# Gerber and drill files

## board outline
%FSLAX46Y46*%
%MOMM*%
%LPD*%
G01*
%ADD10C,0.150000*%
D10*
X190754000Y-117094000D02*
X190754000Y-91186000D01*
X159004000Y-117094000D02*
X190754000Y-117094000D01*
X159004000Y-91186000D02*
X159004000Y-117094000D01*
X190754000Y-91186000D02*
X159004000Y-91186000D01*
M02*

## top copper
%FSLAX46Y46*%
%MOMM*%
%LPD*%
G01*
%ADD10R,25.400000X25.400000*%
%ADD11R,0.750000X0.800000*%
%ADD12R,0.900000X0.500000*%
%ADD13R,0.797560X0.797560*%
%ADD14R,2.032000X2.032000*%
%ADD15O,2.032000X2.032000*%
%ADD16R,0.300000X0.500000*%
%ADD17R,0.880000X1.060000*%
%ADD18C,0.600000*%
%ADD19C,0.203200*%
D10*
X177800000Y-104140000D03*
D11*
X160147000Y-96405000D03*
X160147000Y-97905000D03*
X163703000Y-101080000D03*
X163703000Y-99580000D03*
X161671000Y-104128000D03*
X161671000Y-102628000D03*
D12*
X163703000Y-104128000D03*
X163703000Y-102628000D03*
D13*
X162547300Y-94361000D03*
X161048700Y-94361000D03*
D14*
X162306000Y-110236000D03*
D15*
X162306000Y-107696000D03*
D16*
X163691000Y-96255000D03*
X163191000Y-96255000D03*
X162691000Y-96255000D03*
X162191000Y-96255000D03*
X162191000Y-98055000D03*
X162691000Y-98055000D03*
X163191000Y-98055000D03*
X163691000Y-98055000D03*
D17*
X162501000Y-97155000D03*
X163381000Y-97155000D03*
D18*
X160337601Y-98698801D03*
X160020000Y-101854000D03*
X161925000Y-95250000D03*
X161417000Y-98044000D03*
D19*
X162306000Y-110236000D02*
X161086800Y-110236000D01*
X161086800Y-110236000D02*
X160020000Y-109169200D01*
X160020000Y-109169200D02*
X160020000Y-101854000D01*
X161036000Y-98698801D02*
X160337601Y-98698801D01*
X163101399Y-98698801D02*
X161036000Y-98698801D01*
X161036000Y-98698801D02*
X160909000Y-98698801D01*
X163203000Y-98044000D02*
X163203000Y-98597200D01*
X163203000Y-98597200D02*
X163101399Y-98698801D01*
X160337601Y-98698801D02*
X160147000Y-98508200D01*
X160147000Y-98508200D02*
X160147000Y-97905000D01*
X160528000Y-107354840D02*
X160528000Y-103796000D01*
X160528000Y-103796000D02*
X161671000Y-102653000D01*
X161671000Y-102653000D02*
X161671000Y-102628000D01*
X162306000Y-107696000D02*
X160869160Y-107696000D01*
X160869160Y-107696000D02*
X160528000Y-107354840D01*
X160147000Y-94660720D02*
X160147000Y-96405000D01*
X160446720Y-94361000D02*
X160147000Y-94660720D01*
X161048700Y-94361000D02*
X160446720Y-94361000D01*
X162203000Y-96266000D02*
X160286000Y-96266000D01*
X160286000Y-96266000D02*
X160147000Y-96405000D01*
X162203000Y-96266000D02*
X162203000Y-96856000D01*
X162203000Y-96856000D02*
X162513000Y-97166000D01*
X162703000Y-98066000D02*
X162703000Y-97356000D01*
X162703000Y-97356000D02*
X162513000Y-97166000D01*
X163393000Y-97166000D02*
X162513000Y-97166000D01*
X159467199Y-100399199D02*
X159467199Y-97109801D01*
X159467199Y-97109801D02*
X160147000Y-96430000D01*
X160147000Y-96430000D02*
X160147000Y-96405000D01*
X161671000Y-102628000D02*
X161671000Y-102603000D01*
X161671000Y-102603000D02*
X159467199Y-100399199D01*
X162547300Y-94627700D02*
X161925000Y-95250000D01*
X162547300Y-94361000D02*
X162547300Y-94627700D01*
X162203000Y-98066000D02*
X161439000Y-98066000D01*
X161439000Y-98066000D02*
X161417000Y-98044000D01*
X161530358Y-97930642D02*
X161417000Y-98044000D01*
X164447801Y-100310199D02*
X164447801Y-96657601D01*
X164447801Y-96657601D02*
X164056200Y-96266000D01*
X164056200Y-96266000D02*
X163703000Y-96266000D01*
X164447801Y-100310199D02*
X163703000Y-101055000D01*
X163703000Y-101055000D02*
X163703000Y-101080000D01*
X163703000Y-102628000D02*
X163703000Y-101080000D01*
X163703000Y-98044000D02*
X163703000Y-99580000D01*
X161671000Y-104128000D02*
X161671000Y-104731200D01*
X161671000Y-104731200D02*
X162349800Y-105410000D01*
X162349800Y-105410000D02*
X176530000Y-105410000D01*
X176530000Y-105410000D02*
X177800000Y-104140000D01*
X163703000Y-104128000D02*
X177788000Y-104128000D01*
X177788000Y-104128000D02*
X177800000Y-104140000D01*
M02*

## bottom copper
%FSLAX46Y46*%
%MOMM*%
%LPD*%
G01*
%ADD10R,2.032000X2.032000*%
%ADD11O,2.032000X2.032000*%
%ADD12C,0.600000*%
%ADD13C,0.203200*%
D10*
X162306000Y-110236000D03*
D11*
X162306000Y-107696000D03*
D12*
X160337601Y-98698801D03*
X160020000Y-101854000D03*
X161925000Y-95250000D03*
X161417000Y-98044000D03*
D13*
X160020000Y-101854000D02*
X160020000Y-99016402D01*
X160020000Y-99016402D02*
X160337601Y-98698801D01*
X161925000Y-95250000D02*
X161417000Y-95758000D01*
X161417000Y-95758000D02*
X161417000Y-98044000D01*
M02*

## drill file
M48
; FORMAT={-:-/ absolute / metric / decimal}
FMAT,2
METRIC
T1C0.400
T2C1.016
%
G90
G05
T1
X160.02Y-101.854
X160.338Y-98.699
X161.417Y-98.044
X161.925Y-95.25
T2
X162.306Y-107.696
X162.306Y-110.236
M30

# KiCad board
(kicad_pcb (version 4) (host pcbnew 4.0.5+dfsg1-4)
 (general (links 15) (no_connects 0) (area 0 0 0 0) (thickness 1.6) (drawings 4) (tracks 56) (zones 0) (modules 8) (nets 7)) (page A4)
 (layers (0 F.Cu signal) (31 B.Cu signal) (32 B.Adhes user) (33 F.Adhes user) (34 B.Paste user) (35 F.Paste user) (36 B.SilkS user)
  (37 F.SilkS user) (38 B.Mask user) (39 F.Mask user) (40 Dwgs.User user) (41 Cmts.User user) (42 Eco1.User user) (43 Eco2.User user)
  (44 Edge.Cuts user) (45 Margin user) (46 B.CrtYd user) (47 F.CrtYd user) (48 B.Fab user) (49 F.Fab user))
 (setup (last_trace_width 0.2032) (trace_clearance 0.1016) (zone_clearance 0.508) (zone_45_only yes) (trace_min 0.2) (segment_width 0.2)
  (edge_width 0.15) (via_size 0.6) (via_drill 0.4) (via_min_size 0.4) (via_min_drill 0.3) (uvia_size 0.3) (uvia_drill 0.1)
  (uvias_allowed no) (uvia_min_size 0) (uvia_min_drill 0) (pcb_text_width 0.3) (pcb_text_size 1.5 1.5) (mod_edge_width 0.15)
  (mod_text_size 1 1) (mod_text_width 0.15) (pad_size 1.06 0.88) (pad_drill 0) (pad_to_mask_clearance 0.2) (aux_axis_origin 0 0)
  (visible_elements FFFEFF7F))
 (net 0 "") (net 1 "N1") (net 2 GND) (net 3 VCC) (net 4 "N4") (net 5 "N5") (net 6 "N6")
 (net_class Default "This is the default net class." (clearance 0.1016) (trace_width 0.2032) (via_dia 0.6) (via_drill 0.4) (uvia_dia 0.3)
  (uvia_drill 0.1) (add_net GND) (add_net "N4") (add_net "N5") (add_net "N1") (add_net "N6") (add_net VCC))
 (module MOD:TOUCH (layer F.Cu) (at 177.8 104.14)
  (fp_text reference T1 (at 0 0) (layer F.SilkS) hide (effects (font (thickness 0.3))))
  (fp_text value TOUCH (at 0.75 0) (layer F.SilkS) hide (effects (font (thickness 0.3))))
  (pad 1 connect rect (at 0 0) (size 25.4 25.4) (layers F.Cu) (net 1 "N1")))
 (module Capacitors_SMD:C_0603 (layer F.Cu) (at 160.147 97.155 270)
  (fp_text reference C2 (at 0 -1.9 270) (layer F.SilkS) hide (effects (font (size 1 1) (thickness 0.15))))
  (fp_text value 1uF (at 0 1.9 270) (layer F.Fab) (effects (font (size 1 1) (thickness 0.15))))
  (pad 1 smd rect (at -0.75 0 270) (size 0.8 0.75) (layers F.Cu F.Paste F.Mask) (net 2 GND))
  (pad 2 smd rect (at 0.75 0 270) (size 0.8 0.75) (layers F.Cu F.Paste F.Mask) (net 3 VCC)))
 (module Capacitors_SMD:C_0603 (layer F.Cu) (at 163.703 100.33 90)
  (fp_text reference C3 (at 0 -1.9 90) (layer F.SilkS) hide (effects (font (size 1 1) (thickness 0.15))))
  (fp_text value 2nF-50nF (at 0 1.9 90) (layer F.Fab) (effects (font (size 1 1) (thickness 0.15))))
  (pad 1 smd rect (at -0.75 0 90) (size 0.8 0.75) (layers F.Cu F.Paste F.Mask) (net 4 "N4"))
  (pad 2 smd rect (at 0.75 0 90) (size 0.8 0.75) (layers F.Cu F.Paste F.Mask) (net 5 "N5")))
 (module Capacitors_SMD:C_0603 (layer F.Cu) (at 161.671 103.378 90)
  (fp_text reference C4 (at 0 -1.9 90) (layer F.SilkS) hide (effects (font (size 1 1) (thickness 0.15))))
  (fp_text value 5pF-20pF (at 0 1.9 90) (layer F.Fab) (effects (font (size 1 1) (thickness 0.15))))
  (pad 1 smd rect (at -0.75 0 90) (size 0.8 0.75) (layers F.Cu F.Paste F.Mask) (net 1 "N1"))
  (pad 2 smd rect (at 0.75 0 90) (size 0.8 0.75) (layers F.Cu F.Paste F.Mask) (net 2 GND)))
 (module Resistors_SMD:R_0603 (layer F.Cu) (at 163.703 103.378 90)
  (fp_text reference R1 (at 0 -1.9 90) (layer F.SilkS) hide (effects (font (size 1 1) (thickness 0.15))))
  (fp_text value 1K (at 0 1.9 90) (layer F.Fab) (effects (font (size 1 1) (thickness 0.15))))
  (pad 1 smd rect (at -0.75 0 90) (size 0.5 0.9) (layers F.Cu F.Paste F.Mask) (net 1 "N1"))
  (pad 2 smd rect (at 0.75 0 90) (size 0.5 0.9) (layers F.Cu F.Paste F.Mask) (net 4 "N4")))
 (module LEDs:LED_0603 (layer F.Cu) (at 161.798 94.361)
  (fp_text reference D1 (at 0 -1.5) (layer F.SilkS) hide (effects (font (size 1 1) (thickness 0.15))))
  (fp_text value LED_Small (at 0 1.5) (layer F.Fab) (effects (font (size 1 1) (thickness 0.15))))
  (pad 2 smd rect (at 0.7493 0 180) (size 0.79756 0.79756) (layers F.Cu F.Paste F.Mask) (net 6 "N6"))
  (pad 1 smd rect (at -0.7493 0 180) (size 0.79756 0.79756) (layers F.Cu F.Paste F.Mask) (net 2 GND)))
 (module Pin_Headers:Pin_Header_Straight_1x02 (layer F.Cu) (at 162.306 110.236 180)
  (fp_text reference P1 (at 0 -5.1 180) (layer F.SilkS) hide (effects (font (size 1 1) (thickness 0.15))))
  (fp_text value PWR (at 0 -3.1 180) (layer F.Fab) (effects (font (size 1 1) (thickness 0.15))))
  (pad 1 thru_hole rect (at 0 0 180) (size 2.032 2.032) (drill 1.016) (layers *.Cu *.Mask) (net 3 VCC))
  (pad 2 thru_hole oval (at 0 2.54 180) (size 2.032 2.032) (drill 1.016) (layers *.Cu *.Mask) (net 2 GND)))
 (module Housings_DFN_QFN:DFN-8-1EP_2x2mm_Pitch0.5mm (layer F.Cu) (at 162.941 97.155 270)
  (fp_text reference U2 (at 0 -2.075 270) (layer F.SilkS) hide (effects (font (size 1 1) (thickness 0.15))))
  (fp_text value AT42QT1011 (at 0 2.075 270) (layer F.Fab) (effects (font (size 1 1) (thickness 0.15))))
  (pad 1 smd rect (at -0.9 -0.75 270) (size 0.5 0.3) (layers F.Cu F.Paste F.Mask) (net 4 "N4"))
  (pad 2 smd rect (at -0.9 -0.25 270) (size 0.5 0.3) (layers F.Cu F.Paste F.Mask))
  (pad 3 smd rect (at -0.9 0.25 270) (size 0.5 0.3) (layers F.Cu F.Paste F.Mask))
  (pad 4 smd rect (at -0.9 0.75 270) (size 0.5 0.3) (layers F.Cu F.Paste F.Mask) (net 2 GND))
  (pad 5 smd rect (at 0.9 0.75 270) (size 0.5 0.3) (layers F.Cu F.Paste F.Mask) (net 6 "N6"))
  (pad 6 smd rect (at 0.9 0.25 270) (size 0.5 0.3) (layers F.Cu F.Paste F.Mask) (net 2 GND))
  (pad 7 smd rect (at 0.9 -0.25 270) (size 0.5 0.3) (layers F.Cu F.Paste F.Mask) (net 3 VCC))
  (pad 8 smd rect (at 0.9 -0.75 270) (size 0.5 0.3) (layers F.Cu F.Paste F.Mask) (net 5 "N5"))
  (pad 9 smd rect (at 0 0.44 270) (size 1.06 0.88) (layers F.Cu F.Paste F.Mask) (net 2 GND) (solder_paste_margin_ratio -0.2))
  (pad 9 smd rect (at 0 -0.44 270) (size 1.06 0.88) (layers F.Cu F.Paste F.Mask) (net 2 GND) (solder_paste_margin_ratio -0.2)))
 (gr_line (start 190.754 117.094) (end 190.754 91.186) (layer Edge.Cuts) (width 0.15))
 (gr_line (start 159.004 117.094) (end 190.754 117.094) (layer Edge.Cuts) (width 0.15))
 (gr_line (start 159.004 91.186) (end 159.004 117.094) (layer Edge.Cuts) (width 0.15))
 (gr_line (start 190.754 91.186) (end 159.004 91.186) (layer Edge.Cuts) (width 0.15))
 (segment (start 160.02 101.854) (end 160.02 99.016402) (width 0.2032) (layer B.Cu) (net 3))
 (segment (start 160.02 99.016402) (end 160.337601 98.698801) (width 0.2032) (layer B.Cu) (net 3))
 (via (at 160.337601 98.698801) (size 0.6) (drill 0.4) (layers F.Cu B.Cu) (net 3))
 (segment (start 162.306 110.236) (end 161.0868 110.236) (width 0.2032) (layer F.Cu) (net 3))
 (segment (start 161.0868 110.236) (end 160.02 109.1692) (width 0.2032) (layer F.Cu) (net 3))
 (segment (start 160.02 109.1692) (end 160.02 101.854) (width 0.2032) (layer F.Cu) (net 3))
 (via (at 160.02 101.854) (size 0.6) (drill 0.4) (layers F.Cu B.Cu) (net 3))
 (segment (start 161.036 98.698801) (end 160.337601 98.698801) (width 0.2032) (layer F.Cu) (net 3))
 (segment (start 163.101399 98.698801) (end 161.036 98.698801) (width 0.2032) (layer F.Cu) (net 3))
 (segment (start 161.036 98.698801) (end 160.909 98.698801) (width 0.2032) (layer F.Cu) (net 3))
 (segment (start 163.203 98.044) (end 163.203 98.5972) (width 0.2032) (layer F.Cu) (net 3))
 (segment (start 163.203 98.5972) (end 163.101399 98.698801) (width 0.2032) (layer F.Cu) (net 3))
 (segment (start 160.337601 98.698801) (end 160.147 98.5082) (width 0.2032) (layer F.Cu) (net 3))
 (segment (start 160.147 98.5082) (end 160.147 97.905) (width 0.2032) (layer F.Cu) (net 3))
 (segment (start 160.528 107.35484) (end 160.528 103.796) (width 0.2032) (layer F.Cu) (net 2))
 (segment (start 160.528 103.796) (end 161.671 102.653) (width 0.2032) (layer F.Cu) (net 2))
 (segment (start 161.671 102.653) (end 161.671 102.628) (width 0.2032) (layer F.Cu) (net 2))
 (segment (start 162.306 107.696) (end 160.86916 107.696) (width 0.2032) (layer F.Cu) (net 2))
 (segment (start 160.86916 107.696) (end 160.528 107.35484) (width 0.2032) (layer F.Cu) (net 2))
 (segment (start 160.147 94.66072) (end 160.147 96.405) (width 0.2032) (layer F.Cu) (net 2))
 (segment (start 160.44672 94.361) (end 160.147 94.66072) (width 0.2032) (layer F.Cu) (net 2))
 (segment (start 161.0487 94.361) (end 160.44672 94.361) (width 0.2032) (layer F.Cu) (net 2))
 (segment (start 162.203 96.266) (end 160.286 96.266) (width 0.2032) (layer F.Cu) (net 2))
 (segment (start 160.286 96.266) (end 160.147 96.405) (width 0.2032) (layer F.Cu) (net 2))
 (segment (start 162.203 96.266) (end 162.203 96.856) (width 0.2032) (layer F.Cu) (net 2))
 (segment (start 162.203 96.856) (end 162.513 97.166) (width 0.2032) (layer F.Cu) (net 2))
 (segment (start 162.703 98.066) (end 162.703 97.356) (width 0.2032) (layer F.Cu) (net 2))
 (segment (start 162.703 97.356) (end 162.513 97.166) (width 0.2032) (layer F.Cu) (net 2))
 (segment (start 163.393 97.166) (end 162.513 97.166) (width 0.2032) (layer F.Cu) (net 2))
 (segment (start 159.467199 100.399199) (end 159.467199 97.109801) (width 0.2032) (layer F.Cu) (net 2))
 (segment (start 159.467199 97.109801) (end 160.147 96.43) (width 0.2032) (layer F.Cu) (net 2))
 (segment (start 160.147 96.43) (end 160.147 96.405) (width 0.2032) (layer F.Cu) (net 2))
 (segment (start 161.671 102.628) (end 161.671 102.603) (width 0.2032) (layer F.Cu) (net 2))
 (segment (start 161.671 102.603) (end 159.467199 100.399199) (width 0.2032) (layer F.Cu) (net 2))
 (segment (start 161.925 95.25) (end 161.417 95.758) (width 0.2032) (layer B.Cu) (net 6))
 (via (at 161.925 95.25) (size 0.6) (drill 0.4) (layers F.Cu B.Cu) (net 6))
 (segment (start 162.5473 94.6277) (end 161.925 95.25) (width 0.2032) (layer F.Cu) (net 6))
 (segment (start 161.417 95.758) (end 161.417 98.044) (width 0.2032) (layer B.Cu) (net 6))
 (segment (start 162.5473 94.361) (end 162.5473 94.6277) (width 0.2032) (layer F.Cu) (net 6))
 (segment (start 162.203 98.066) (end 161.439 98.066) (width 0.2032) (layer F.Cu) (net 6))
 (segment (start 161.439 98.066) (end 161.417 98.044) (width 0.2032) (layer F.Cu) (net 6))
 (segment (start 161.530358 97.930642) (end 161.417 98.044) (width 0.2032) (layer F.Cu) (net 6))
 (via (at 161.417 98.044) (size 0.6) (drill 0.4) (layers F.Cu B.Cu) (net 6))
 (segment (start 164.447801 100.310199) (end 164.447801 96.657601) (width 0.2032) (layer F.Cu) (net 4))
 (segment (start 164.447801 96.657601) (end 164.0562 96.266) (width 0.2032) (layer F.Cu) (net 4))
 (segment (start 164.0562 96.266) (end 163.703 96.266) (width 0.2032) (layer F.Cu) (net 4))
 (segment (start 164.447801 100.310199) (end 163.703 101.055) (width 0.2032) (layer F.Cu) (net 4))
 (segment (start 163.703 101.055) (end 163.703 101.08) (width 0.2032) (layer F.Cu) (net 4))
 (segment (start 163.703 102.628) (end 163.703 101.08) (width 0.2032) (layer F.Cu) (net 4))
 (segment (start 163.703 98.044) (end 163.703 99.58) (width 0.2032) (layer F.Cu) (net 5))
 (segment (start 161.671 104.128) (end 161.671 104.7312) (width 0.2032) (layer F.Cu) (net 1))
 (segment (start 161.671 104.7312) (end 162.3498 105.41) (width 0.2032) (layer F.Cu) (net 1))
 (segment (start 162.3498 105.41) (end 176.53 105.41) (width 0.2032) (layer F.Cu) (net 1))
 (segment (start 176.53 105.41) (end 177.8 104.14) (width 0.2032) (layer F.Cu) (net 1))
 (segment (start 163.703 104.128) (end 177.788 104.128) (width 0.2032) (layer F.Cu) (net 1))
 (segment (start 177.788 104.128) (end 177.8 104.14) (width 0.2032) (layer F.Cu) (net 1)))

